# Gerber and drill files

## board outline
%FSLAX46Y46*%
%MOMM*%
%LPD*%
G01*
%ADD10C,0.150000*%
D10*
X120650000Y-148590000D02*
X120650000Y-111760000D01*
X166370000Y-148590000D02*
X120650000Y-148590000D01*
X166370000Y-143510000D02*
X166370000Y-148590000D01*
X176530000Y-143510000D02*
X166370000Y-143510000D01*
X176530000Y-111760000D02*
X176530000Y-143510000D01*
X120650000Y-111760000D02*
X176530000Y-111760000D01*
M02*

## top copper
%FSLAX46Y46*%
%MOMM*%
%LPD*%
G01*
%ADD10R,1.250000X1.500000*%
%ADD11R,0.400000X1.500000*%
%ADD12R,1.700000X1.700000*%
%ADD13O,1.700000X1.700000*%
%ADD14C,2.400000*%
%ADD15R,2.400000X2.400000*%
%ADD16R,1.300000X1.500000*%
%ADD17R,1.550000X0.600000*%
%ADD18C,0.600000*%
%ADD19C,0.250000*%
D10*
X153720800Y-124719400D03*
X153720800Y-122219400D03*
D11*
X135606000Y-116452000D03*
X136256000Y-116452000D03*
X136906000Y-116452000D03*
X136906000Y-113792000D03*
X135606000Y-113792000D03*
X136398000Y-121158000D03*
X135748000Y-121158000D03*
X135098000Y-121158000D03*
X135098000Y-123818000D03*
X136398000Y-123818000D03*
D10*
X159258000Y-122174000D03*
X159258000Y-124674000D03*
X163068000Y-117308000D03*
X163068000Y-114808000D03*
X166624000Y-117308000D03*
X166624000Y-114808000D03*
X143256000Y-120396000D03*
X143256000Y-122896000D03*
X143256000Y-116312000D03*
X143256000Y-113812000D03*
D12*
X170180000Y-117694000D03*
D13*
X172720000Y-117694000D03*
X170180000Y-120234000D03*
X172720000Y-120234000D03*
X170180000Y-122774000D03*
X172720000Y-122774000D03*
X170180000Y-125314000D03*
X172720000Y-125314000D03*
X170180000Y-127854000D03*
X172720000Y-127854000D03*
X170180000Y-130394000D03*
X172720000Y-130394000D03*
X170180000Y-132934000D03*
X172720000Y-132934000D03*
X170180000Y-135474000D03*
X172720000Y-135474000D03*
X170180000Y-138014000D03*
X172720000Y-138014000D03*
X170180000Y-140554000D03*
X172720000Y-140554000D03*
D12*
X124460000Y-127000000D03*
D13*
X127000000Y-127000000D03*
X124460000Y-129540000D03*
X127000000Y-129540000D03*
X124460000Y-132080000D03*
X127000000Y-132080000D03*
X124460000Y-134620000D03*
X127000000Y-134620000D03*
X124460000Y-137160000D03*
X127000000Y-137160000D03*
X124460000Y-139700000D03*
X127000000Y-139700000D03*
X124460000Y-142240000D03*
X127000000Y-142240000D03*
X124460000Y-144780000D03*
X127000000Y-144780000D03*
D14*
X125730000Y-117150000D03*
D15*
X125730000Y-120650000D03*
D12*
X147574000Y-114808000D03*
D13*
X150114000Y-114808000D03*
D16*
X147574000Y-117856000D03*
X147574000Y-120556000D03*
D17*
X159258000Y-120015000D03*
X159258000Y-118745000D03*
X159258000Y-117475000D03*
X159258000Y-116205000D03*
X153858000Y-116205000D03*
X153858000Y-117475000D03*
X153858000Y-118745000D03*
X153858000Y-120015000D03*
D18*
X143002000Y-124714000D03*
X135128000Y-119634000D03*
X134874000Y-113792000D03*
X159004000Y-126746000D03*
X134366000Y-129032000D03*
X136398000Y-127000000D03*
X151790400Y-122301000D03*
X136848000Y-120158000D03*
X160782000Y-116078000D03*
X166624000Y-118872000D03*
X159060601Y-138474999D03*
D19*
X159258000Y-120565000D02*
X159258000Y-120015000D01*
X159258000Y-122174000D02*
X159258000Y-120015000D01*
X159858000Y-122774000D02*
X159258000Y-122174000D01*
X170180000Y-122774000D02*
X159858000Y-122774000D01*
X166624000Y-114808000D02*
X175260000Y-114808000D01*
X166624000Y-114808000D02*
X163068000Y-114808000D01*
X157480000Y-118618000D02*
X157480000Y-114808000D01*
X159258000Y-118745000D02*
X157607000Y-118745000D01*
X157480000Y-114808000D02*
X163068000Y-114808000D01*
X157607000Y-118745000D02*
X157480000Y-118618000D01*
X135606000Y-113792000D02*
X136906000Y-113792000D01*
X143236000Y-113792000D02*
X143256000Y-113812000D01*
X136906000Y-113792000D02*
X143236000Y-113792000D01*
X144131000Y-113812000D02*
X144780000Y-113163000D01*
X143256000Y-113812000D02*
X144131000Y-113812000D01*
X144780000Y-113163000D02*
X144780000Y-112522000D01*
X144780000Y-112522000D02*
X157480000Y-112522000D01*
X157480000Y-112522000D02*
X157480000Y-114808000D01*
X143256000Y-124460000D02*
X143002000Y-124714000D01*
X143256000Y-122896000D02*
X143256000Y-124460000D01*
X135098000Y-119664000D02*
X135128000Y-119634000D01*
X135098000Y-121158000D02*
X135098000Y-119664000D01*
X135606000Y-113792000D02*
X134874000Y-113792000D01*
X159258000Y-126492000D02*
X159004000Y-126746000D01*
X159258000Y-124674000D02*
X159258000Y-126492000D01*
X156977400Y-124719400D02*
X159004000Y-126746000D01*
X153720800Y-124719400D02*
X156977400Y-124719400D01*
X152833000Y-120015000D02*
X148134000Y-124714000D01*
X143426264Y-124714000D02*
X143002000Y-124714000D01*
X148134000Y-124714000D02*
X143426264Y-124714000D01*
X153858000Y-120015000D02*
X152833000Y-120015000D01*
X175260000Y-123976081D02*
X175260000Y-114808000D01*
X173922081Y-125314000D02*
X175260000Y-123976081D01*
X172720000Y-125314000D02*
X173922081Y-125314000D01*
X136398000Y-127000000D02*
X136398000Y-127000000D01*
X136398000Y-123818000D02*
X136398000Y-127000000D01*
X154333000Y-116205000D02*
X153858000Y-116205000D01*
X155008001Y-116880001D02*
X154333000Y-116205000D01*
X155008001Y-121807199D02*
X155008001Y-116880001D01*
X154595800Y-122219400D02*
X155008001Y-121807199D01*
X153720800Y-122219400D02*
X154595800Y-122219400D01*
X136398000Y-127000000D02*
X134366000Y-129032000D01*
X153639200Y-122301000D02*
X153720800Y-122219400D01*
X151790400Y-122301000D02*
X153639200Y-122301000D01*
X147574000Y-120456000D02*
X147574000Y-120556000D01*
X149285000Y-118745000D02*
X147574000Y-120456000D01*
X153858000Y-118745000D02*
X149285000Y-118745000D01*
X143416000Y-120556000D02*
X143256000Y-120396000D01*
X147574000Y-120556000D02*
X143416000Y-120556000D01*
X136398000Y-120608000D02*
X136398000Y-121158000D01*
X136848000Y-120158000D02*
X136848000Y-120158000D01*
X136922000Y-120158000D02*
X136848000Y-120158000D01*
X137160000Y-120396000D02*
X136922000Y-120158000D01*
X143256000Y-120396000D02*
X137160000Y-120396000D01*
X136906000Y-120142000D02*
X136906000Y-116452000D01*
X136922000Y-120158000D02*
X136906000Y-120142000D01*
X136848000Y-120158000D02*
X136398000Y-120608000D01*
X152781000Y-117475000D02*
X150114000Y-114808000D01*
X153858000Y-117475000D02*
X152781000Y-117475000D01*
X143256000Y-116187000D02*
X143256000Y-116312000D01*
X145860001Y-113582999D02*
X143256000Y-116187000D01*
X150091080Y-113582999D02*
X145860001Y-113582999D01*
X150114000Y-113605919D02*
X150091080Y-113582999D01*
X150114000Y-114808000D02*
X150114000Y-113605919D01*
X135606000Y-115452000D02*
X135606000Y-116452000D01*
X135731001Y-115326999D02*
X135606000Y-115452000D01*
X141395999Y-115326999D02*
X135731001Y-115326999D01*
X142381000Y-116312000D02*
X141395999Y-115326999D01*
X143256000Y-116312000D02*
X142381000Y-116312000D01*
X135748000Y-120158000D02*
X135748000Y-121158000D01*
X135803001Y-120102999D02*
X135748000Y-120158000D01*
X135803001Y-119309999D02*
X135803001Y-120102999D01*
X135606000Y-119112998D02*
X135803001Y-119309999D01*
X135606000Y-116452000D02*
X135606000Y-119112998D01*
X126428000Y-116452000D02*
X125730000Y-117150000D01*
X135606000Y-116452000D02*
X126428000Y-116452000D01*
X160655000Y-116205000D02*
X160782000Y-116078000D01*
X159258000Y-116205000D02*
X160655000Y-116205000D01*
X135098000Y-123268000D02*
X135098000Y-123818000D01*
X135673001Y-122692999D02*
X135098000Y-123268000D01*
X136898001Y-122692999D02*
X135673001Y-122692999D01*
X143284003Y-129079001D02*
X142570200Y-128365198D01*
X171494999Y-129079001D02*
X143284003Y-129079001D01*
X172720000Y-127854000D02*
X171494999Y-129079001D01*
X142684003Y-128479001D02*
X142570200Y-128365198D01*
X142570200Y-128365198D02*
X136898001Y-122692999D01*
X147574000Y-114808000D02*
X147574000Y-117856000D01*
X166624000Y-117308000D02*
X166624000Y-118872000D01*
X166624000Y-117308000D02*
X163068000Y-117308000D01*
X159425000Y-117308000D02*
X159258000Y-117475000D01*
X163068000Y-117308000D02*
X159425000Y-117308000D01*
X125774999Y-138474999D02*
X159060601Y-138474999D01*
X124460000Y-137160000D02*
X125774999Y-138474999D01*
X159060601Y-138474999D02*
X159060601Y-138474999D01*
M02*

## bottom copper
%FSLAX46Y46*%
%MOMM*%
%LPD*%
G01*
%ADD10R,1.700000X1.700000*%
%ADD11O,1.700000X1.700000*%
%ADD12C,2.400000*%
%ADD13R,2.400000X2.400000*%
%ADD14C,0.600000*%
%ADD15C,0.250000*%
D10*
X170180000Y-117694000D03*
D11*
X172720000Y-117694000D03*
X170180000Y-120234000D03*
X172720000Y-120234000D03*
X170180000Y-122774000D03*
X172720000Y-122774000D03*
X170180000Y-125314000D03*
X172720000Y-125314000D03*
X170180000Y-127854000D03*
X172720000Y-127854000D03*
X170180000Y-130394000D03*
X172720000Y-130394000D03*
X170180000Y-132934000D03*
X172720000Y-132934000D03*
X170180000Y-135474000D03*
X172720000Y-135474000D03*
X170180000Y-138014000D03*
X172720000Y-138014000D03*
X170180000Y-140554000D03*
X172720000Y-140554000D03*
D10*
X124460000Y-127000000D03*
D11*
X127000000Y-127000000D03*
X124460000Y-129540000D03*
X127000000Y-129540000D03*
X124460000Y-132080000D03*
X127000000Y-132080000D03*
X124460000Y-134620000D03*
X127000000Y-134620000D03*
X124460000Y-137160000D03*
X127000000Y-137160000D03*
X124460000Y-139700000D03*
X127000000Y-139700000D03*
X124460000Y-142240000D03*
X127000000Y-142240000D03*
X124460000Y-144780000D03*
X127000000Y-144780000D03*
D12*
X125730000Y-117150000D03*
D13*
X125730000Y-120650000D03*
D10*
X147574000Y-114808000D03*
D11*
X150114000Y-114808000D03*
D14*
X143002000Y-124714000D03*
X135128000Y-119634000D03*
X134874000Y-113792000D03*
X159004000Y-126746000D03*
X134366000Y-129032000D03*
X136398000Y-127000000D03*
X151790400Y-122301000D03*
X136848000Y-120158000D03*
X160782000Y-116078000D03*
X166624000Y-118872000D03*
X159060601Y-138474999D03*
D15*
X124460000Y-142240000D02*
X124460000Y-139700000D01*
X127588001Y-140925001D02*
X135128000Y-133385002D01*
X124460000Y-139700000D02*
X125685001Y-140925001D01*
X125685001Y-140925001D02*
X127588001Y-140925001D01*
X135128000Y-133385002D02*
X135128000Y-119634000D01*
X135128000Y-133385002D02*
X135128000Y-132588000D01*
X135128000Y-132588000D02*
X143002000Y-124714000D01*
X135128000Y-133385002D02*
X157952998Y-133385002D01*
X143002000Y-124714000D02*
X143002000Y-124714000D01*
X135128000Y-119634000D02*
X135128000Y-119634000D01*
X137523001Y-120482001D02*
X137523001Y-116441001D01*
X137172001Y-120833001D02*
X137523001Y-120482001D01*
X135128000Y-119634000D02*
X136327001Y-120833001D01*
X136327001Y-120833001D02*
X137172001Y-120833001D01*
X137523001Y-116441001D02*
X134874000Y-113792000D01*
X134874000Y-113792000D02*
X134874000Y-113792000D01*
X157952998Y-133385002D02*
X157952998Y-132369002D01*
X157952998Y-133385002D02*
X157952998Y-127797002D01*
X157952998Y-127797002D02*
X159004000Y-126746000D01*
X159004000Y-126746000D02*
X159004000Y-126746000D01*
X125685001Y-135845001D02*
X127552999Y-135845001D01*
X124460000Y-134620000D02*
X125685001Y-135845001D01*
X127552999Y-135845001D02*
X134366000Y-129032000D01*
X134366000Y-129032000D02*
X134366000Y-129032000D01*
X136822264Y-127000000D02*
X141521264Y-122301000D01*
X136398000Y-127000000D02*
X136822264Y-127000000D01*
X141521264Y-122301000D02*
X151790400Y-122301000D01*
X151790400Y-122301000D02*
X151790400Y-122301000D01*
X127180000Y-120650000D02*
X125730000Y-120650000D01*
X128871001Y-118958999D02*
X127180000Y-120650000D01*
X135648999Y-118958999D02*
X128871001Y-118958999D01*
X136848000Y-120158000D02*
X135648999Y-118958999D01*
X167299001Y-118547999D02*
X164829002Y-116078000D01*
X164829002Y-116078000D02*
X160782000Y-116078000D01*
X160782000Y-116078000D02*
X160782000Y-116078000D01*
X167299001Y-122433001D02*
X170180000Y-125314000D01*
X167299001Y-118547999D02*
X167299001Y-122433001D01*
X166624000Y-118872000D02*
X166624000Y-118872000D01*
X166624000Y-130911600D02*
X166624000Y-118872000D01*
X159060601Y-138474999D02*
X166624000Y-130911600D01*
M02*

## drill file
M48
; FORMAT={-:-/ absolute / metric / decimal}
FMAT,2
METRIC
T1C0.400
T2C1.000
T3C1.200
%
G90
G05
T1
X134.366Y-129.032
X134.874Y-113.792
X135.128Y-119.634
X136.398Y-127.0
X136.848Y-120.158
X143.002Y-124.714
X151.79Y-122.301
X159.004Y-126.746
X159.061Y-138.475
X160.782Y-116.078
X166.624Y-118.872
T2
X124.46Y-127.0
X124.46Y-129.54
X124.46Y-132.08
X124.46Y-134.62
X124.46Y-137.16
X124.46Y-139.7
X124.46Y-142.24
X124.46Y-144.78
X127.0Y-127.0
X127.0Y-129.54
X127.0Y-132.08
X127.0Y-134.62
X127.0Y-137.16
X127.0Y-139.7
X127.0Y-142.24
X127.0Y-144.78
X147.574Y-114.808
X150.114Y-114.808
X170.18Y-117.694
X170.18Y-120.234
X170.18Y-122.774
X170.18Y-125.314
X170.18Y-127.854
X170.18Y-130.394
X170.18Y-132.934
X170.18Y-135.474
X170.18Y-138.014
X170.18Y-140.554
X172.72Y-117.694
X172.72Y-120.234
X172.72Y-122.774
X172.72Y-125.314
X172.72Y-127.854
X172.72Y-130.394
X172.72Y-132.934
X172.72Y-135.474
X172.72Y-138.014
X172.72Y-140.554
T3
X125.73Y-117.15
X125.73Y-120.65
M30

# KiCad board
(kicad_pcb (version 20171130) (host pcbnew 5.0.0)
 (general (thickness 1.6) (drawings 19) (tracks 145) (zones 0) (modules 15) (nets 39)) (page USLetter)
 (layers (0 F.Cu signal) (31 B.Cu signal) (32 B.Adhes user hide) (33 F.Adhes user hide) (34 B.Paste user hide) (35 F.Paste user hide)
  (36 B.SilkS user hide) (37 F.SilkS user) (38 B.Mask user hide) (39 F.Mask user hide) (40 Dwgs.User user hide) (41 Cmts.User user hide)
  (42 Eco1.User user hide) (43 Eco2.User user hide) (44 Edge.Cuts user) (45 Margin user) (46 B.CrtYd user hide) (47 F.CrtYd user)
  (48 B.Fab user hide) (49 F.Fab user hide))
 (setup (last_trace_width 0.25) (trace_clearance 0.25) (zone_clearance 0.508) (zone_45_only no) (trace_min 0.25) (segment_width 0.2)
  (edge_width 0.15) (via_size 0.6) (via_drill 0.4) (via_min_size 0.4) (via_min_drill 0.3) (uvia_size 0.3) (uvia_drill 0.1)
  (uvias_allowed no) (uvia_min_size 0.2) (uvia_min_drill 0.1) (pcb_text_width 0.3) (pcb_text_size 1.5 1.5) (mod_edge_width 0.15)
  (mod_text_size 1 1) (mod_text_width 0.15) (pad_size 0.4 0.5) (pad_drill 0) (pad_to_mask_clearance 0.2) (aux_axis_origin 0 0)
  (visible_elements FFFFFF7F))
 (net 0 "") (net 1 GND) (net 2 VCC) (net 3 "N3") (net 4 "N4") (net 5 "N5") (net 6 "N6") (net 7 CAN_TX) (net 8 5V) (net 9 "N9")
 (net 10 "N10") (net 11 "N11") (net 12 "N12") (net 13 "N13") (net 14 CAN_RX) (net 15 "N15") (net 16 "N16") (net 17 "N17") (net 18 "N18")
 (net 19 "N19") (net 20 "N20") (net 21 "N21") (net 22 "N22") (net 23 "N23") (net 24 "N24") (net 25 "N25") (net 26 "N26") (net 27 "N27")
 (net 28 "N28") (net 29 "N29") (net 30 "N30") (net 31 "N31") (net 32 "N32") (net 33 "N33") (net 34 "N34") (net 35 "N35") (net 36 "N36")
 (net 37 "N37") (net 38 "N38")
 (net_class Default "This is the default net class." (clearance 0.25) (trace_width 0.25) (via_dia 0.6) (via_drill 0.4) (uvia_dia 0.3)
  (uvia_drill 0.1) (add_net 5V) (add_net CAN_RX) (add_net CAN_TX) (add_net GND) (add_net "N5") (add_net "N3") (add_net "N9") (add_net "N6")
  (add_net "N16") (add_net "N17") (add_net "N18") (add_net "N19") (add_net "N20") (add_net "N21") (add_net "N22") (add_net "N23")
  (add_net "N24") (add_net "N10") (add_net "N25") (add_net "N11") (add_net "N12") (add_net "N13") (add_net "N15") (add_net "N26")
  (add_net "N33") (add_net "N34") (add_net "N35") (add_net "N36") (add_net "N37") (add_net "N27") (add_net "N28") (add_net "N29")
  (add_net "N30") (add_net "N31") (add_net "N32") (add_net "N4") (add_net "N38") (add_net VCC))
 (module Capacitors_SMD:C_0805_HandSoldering (layer F.Cu) (at 153.7208 123.4694 90)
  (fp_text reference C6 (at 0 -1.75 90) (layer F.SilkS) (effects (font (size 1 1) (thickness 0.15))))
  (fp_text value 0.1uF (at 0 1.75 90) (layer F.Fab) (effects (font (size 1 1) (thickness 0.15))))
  (pad 1 smd rect (at -1.25 0 90) (size 1.5 1.25) (layers F.Cu F.Paste F.Mask) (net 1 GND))
  (pad 2 smd rect (at 1.25 0 90) (size 1.5 1.25) (layers F.Cu F.Paste F.Mask) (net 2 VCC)))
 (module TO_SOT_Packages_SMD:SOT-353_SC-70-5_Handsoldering (layer F.Cu) (at 136.256 115.122 90)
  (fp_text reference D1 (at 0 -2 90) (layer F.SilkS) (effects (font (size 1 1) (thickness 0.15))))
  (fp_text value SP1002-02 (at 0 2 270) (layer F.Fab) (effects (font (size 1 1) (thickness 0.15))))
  (pad 1 smd rect (at -1.33 -0.65 90) (size 1.5 0.4) (layers F.Cu F.Paste F.Mask) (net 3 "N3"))
  (pad 2 smd rect (at -1.33 0 90) (size 1.5 0.4) (layers F.Cu F.Paste F.Mask) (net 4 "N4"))
  (pad 3 smd rect (at -1.33 0.65 90) (size 1.5 0.4) (layers F.Cu F.Paste F.Mask) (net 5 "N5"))
  (pad 4 smd rect (at 1.33 0.65 90) (size 1.5 0.4) (layers F.Cu F.Paste F.Mask) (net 1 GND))
  (pad 5 smd rect (at 1.33 -0.65 90) (size 1.5 0.4) (layers F.Cu F.Paste F.Mask) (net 1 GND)))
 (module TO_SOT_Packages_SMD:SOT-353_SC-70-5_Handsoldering (layer F.Cu) (at 135.748 122.488 270)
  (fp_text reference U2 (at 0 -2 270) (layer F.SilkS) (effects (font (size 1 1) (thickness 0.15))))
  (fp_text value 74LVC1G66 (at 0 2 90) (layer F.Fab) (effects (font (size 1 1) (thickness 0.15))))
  (pad 1 smd rect (at -1.33 -0.65 270) (size 1.5 0.4) (layers F.Cu F.Paste F.Mask) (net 5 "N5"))
  (pad 2 smd rect (at -1.33 0 270) (size 1.5 0.4) (layers F.Cu F.Paste F.Mask) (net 3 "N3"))
  (pad 3 smd rect (at -1.33 0.65 270) (size 1.5 0.4) (layers F.Cu F.Paste F.Mask) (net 1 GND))
  (pad 4 smd rect (at 1.33 0.65 270) (size 1.5 0.4) (layers F.Cu F.Paste F.Mask) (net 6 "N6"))
  (pad 5 smd rect (at 1.33 -0.65 270) (size 1.5 0.4) (layers F.Cu F.Paste F.Mask) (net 2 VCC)))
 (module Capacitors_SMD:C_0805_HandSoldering (layer F.Cu) (at 159.258 123.424 270)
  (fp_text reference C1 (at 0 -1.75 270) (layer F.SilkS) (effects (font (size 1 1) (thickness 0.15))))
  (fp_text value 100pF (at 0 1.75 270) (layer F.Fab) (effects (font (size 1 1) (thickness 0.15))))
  (pad 1 smd rect (at -1.25 0 270) (size 1.5 1.25) (layers F.Cu F.Paste F.Mask) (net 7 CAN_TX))
  (pad 2 smd rect (at 1.25 0 270) (size 1.5 1.25) (layers F.Cu F.Paste F.Mask) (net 1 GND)))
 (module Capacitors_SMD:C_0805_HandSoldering (layer F.Cu) (at 163.068 116.058 90)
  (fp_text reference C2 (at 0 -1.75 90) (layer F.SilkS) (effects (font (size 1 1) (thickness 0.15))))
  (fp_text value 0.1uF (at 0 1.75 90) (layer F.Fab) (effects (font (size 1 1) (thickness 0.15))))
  (pad 1 smd rect (at -1.25 0 90) (size 1.5 1.25) (layers F.Cu F.Paste F.Mask) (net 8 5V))
  (pad 2 smd rect (at 1.25 0 90) (size 1.5 1.25) (layers F.Cu F.Paste F.Mask) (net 1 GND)))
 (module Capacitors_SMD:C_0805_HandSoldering (layer F.Cu) (at 166.624 116.058 90)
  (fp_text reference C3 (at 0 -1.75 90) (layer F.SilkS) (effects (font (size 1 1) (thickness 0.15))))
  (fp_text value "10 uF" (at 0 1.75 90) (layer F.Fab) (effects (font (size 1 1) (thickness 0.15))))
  (pad 1 smd rect (at -1.25 0 90) (size 1.5 1.25) (layers F.Cu F.Paste F.Mask) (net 8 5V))
  (pad 2 smd rect (at 1.25 0 90) (size 1.5 1.25) (layers F.Cu F.Paste F.Mask) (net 1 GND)))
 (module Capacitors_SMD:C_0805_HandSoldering (layer F.Cu) (at 143.256 121.646 270)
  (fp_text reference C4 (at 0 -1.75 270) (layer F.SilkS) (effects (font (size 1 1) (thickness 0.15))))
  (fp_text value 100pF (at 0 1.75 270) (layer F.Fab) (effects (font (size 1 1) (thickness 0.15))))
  (pad 1 smd rect (at -1.25 0 270) (size 1.5 1.25) (layers F.Cu F.Paste F.Mask) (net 5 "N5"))
  (pad 2 smd rect (at 1.25 0 270) (size 1.5 1.25) (layers F.Cu F.Paste F.Mask) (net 1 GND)))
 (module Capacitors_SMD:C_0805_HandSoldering (layer F.Cu) (at 143.256 115.062 90)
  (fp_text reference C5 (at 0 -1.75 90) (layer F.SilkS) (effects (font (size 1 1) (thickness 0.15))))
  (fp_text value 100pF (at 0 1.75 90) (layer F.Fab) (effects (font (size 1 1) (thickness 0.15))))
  (pad 1 smd rect (at -1.25 0 90) (size 1.5 1.25) (layers F.Cu F.Paste F.Mask) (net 3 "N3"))
  (pad 2 smd rect (at 1.25 0 90) (size 1.5 1.25) (layers F.Cu F.Paste F.Mask) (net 1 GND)))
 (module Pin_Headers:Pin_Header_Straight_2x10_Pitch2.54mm (layer F.Cu) (at 170.18 117.694)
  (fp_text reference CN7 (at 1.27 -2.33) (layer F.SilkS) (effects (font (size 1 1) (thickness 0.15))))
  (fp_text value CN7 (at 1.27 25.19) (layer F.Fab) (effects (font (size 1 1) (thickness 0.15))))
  (pad 1 thru_hole rect (at 0 0) (size 1.7 1.7) (drill 1) (layers *.Cu *.Mask) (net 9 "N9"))
  (pad 2 thru_hole oval (at 2.54 0) (size 1.7 1.7) (drill 1) (layers *.Cu *.Mask) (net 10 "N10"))
  (pad 3 thru_hole oval (at 0 2.54) (size 1.7 1.7) (drill 1) (layers *.Cu *.Mask) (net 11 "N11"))
  (pad 4 thru_hole oval (at 2.54 2.54) (size 1.7 1.7) (drill 1) (layers *.Cu *.Mask) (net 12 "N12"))
  (pad 5 thru_hole oval (at 0 5.08) (size 1.7 1.7) (drill 1) (layers *.Cu *.Mask) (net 7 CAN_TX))
  (pad 6 thru_hole oval (at 2.54 5.08) (size 1.7 1.7) (drill 1) (layers *.Cu *.Mask) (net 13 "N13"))
  (pad 7 thru_hole oval (at 0 7.62) (size 1.7 1.7) (drill 1) (layers *.Cu *.Mask) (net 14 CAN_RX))
  (pad 8 thru_hole oval (at 2.54 7.62) (size 1.7 1.7) (drill 1) (layers *.Cu *.Mask) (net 1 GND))
  (pad 9 thru_hole oval (at 0 10.16) (size 1.7 1.7) (drill 1) (layers *.Cu *.Mask) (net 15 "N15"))
  (pad 10 thru_hole oval (at 2.54 10.16) (size 1.7 1.7) (drill 1) (layers *.Cu *.Mask) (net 6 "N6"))
  (pad 11 thru_hole oval (at 0 12.7) (size 1.7 1.7) (drill 1) (layers *.Cu *.Mask) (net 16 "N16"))
  (pad 12 thru_hole oval (at 2.54 12.7) (size 1.7 1.7) (drill 1) (layers *.Cu *.Mask) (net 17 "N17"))
  (pad 13 thru_hole oval (at 0 15.24) (size 1.7 1.7) (drill 1) (layers *.Cu *.Mask) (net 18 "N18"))
  (pad 14 thru_hole oval (at 2.54 15.24) (size 1.7 1.7) (drill 1) (layers *.Cu *.Mask) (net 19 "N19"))
  (pad 15 thru_hole oval (at 0 17.78) (size 1.7 1.7) (drill 1) (layers *.Cu *.Mask) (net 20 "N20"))
  (pad 16 thru_hole oval (at 2.54 17.78) (size 1.7 1.7) (drill 1) (layers *.Cu *.Mask) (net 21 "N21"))
  (pad 17 thru_hole oval (at 0 20.32) (size 1.7 1.7) (drill 1) (layers *.Cu *.Mask) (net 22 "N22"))
  (pad 18 thru_hole oval (at 2.54 20.32) (size 1.7 1.7) (drill 1) (layers *.Cu *.Mask) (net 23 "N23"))
  (pad 19 thru_hole oval (at 0 22.86) (size 1.7 1.7) (drill 1) (layers *.Cu *.Mask) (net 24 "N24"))
  (pad 20 thru_hole oval (at 2.54 22.86) (size 1.7 1.7) (drill 1) (layers *.Cu *.Mask) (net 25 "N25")))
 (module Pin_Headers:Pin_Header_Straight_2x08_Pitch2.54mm (layer F.Cu) (at 124.46 127)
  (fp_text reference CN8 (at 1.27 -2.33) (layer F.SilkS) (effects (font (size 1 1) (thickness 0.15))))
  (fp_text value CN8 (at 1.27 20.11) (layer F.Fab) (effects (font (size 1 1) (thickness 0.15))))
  (pad 1 thru_hole rect (at 0 0) (size 1.7 1.7) (drill 1) (layers *.Cu *.Mask) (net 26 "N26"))
  (pad 2 thru_hole oval (at 2.54 0) (size 1.7 1.7) (drill 1) (layers *.Cu *.Mask) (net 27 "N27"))
  (pad 3 thru_hole oval (at 0 2.54) (size 1.7 1.7) (drill 1) (layers *.Cu *.Mask) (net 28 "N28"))
  (pad 4 thru_hole oval (at 2.54 2.54) (size 1.7 1.7) (drill 1) (layers *.Cu *.Mask) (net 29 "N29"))
  (pad 5 thru_hole oval (at 0 5.08) (size 1.7 1.7) (drill 1) (layers *.Cu *.Mask) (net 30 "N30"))
  (pad 6 thru_hole oval (at 2.54 5.08) (size 1.7 1.7) (drill 1) (layers *.Cu *.Mask) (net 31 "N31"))
  (pad 7 thru_hole oval (at 0 7.62) (size 1.7 1.7) (drill 1) (layers *.Cu *.Mask) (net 2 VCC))
  (pad 8 thru_hole oval (at 2.54 7.62) (size 1.7 1.7) (drill 1) (layers *.Cu *.Mask) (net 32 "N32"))
  (pad 9 thru_hole oval (at 0 10.16) (size 1.7 1.7) (drill 1) (layers *.Cu *.Mask) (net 8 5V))
  (pad 10 thru_hole oval (at 2.54 10.16) (size 1.7 1.7) (drill 1) (layers *.Cu *.Mask) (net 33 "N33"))
  (pad 11 thru_hole oval (at 0 12.7) (size 1.7 1.7) (drill 1) (layers *.Cu *.Mask) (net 1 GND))
  (pad 12 thru_hole oval (at 2.54 12.7) (size 1.7 1.7) (drill 1) (layers *.Cu *.Mask) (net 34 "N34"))
  (pad 13 thru_hole oval (at 0 15.24) (size 1.7 1.7) (drill 1) (layers *.Cu *.Mask) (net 1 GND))
  (pad 14 thru_hole oval (at 2.54 15.24) (size 1.7 1.7) (drill 1) (layers *.Cu *.Mask) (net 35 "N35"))
  (pad 15 thru_hole oval (at 0 17.78) (size 1.7 1.7) (drill 1) (layers *.Cu *.Mask) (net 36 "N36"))
  (pad 16 thru_hole oval (at 2.54 17.78) (size 1.7 1.7) (drill 1) (layers *.Cu *.Mask) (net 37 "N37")))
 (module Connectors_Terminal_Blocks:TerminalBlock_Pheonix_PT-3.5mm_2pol (layer F.Cu) (at 125.73 120.65 90)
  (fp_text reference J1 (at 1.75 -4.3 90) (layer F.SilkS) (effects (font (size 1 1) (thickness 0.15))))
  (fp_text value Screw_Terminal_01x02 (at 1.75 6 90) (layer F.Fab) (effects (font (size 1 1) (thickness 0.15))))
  (pad 2 thru_hole circle (at 3.5 0 90) (size 2.4 2.4) (drill 1.2) (layers *.Cu *.Mask) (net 3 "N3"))
  (pad 1 thru_hole rect (at 0 0 90) (size 2.4 2.4) (drill 1.2) (layers *.Cu *.Mask) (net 5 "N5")))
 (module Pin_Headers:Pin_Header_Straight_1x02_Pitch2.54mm (layer F.Cu) (at 147.574 114.808 90)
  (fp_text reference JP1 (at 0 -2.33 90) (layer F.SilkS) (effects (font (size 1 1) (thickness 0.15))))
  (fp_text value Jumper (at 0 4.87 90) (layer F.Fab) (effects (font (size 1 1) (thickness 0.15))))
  (pad 1 thru_hole rect (at 0 0 90) (size 1.7 1.7) (drill 1) (layers *.Cu *.Mask) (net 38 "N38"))
  (pad 2 thru_hole oval (at 0 2.54 90) (size 1.7 1.7) (drill 1) (layers *.Cu *.Mask) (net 3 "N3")))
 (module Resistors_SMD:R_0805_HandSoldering (layer F.Cu) (at 147.574 119.206 270)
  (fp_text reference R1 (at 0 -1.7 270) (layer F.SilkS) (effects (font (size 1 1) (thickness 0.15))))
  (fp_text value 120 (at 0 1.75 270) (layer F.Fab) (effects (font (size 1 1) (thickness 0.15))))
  (pad 1 smd rect (at -1.35 0 270) (size 1.5 1.3) (layers F.Cu F.Paste F.Mask) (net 38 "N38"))
  (pad 2 smd rect (at 1.35 0 270) (size 1.5 1.3) (layers F.Cu F.Paste F.Mask) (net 5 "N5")))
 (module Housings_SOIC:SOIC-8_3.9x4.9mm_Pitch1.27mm (layer F.Cu) (at 156.558 118.11 180)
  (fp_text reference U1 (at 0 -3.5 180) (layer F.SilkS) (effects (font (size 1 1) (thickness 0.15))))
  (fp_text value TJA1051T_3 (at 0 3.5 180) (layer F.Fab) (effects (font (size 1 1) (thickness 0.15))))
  (pad 1 smd rect (at -2.7 -1.905 180) (size 1.55 0.6) (layers F.Cu F.Paste F.Mask) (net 7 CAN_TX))
  (pad 2 smd rect (at -2.7 -0.635 180) (size 1.55 0.6) (layers F.Cu F.Paste F.Mask) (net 1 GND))
  (pad 3 smd rect (at -2.7 0.635 180) (size 1.55 0.6) (layers F.Cu F.Paste F.Mask) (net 8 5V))
  (pad 4 smd rect (at -2.7 1.905 180) (size 1.55 0.6) (layers F.Cu F.Paste F.Mask) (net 14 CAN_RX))
  (pad 5 smd rect (at 2.7 1.905 180) (size 1.55 0.6) (layers F.Cu F.Paste F.Mask) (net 2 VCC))
  (pad 6 smd rect (at 2.7 0.635 180) (size 1.55 0.6) (layers F.Cu F.Paste F.Mask) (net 3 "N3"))
  (pad 7 smd rect (at 2.7 -0.635 180) (size 1.55 0.6) (layers F.Cu F.Paste F.Mask) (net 5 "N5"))
  (pad 8 smd rect (at 2.7 -1.905 180) (size 1.55 0.6) (layers F.Cu F.Paste F.Mask) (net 1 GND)))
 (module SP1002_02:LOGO (layer B.Cu) (at 147.32 134.2898)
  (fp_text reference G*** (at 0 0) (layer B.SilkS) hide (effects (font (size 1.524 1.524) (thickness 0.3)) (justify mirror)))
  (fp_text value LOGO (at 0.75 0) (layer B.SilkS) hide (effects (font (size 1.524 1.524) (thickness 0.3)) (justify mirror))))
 (gr_line (start 120.65 148.59) (end 120.65 111.76) (angle 90) (layer Edge.Cuts) (width 0.15))
 (gr_line (start 166.37 148.59) (end 120.65 148.59) (angle 90) (layer Edge.Cuts) (width 0.15))
 (gr_line (start 166.37 143.51) (end 166.37 148.59) (angle 90) (layer Edge.Cuts) (width 0.15))
 (gr_line (start 176.53 143.51) (end 166.37 143.51) (angle 90) (layer Edge.Cuts) (width 0.15))
 (gr_line (start 176.53 111.76) (end 176.53 143.51) (angle 90) (layer Edge.Cuts) (width 0.15))
 (gr_line (start 120.65 111.76) (end 176.53 111.76) (angle 90) (layer Edge.Cuts) (width 0.15))
 (segment (start 159.258 120.565) (end 159.258 120.015) (width 0.25) (layer F.Cu) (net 7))
 (segment (start 159.258 122.174) (end 159.258 120.015) (width 0.25) (layer F.Cu) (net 7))
 (segment (start 159.858 122.774) (end 159.258 122.174) (width 0.25) (layer F.Cu) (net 7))
 (segment (start 170.18 122.774) (end 159.858 122.774) (width 0.25) (layer F.Cu) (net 7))
 (segment (start 124.46 142.24) (end 124.46 139.7) (width 0.25) (layer B.Cu) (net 1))
 (segment (start 166.624 114.808) (end 175.26 114.808) (width 0.25) (layer F.Cu) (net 1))
 (segment (start 166.624 114.808) (end 163.068 114.808) (width 0.25) (layer F.Cu) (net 1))
 (segment (start 157.48 118.618) (end 157.48 114.808) (width 0.25) (layer F.Cu) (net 1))
 (segment (start 159.258 118.745) (end 157.607 118.745) (width 0.25) (layer F.Cu) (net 1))
 (segment (start 157.48 114.808) (end 163.068 114.808) (width 0.25) (layer F.Cu) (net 1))
 (segment (start 157.607 118.745) (end 157.48 118.618) (width 0.25) (layer F.Cu) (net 1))
 (segment (start 135.606 113.792) (end 136.906 113.792) (width 0.25) (layer F.Cu) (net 1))
 (segment (start 143.236 113.792) (end 143.256 113.812) (width 0.25) (layer F.Cu) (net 1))
 (segment (start 136.906 113.792) (end 143.236 113.792) (width 0.25) (layer F.Cu) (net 1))
 (segment (start 144.131 113.812) (end 144.78 113.163) (width 0.25) (layer F.Cu) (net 1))
 (segment (start 143.256 113.812) (end 144.131 113.812) (width 0.25) (layer F.Cu) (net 1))
 (segment (start 144.78 113.163) (end 144.78 112.522) (width 0.25) (layer F.Cu) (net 1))
 (segment (start 144.78 112.522) (end 157.48 112.522) (width 0.25) (layer F.Cu) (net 1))
 (segment (start 157.48 112.522) (end 157.48 114.808) (width 0.25) (layer F.Cu) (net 1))
 (segment (start 127.588001 140.925001) (end 135.128 133.385002) (width 0.25) (layer B.Cu) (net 1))
 (segment (start 124.46 139.7) (end 125.685001 140.925001) (width 0.25) (layer B.Cu) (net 1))
 (segment (start 125.685001 140.925001) (end 127.588001 140.925001) (width 0.25) (layer B.Cu) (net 1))
 (segment (start 135.128 133.385002) (end 135.128 119.634) (width 0.25) (layer B.Cu) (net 1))
 (segment (start 135.128 133.385002) (end 135.128 132.588) (width 0.25) (layer B.Cu) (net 1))
 (segment (start 135.128 132.588) (end 143.002 124.714) (width 0.25) (layer B.Cu) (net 1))
 (segment (start 135.128 133.385002) (end 157.952998 133.385002) (width 0.25) (layer B.Cu) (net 1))
 (segment (start 143.002 124.714) (end 143.002 124.714) (width 0.25) (layer B.Cu) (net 1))
 (via (at 143.002 124.714) (size 0.6) (drill 0.4) (layers F.Cu B.Cu) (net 1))
 (segment (start 135.128 119.634) (end 135.128 119.634) (width 0.25) (layer B.Cu) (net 1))
 (via (at 135.128 119.634) (size 0.6) (drill 0.4) (layers F.Cu B.Cu) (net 1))
 (segment (start 143.256 124.46) (end 143.002 124.714) (width 0.25) (layer F.Cu) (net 1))
 (segment (start 143.256 122.896) (end 143.256 124.46) (width 0.25) (layer F.Cu) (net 1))
 (segment (start 135.098 119.664) (end 135.128 119.634) (width 0.25) (layer F.Cu) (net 1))
 (segment (start 135.098 121.158) (end 135.098 119.664) (width 0.25) (layer F.Cu) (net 1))
 (segment (start 137.523001 120.482001) (end 137.523001 116.441001) (width 0.25) (layer B.Cu) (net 1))
 (segment (start 137.172001 120.833001) (end 137.523001 120.482001) (width 0.25) (layer B.Cu) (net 1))
 (segment (start 135.128 119.634) (end 136.327001 120.833001) (width 0.25) (layer B.Cu) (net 1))
 (segment (start 136.327001 120.833001) (end 137.172001 120.833001) (width 0.25) (layer B.Cu) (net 1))
 (segment (start 137.523001 116.441001) (end 134.874 113.792) (width 0.25) (layer B.Cu) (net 1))
 (segment (start 134.874 113.792) (end 134.874 113.792) (width 0.25) (layer B.Cu) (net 1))
 (via (at 134.874 113.792) (size 0.6) (drill 0.4) (layers F.Cu B.Cu) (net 1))
 (segment (start 135.606 113.792) (end 134.874 113.792) (width 0.25) (layer F.Cu) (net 1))
 (segment (start 157.952998 133.385002) (end 157.952998 132.369002) (width 0.25) (layer B.Cu) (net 1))
 (segment (start 157.952998 133.385002) (end 157.952998 127.797002) (width 0.25) (layer B.Cu) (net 1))
 (segment (start 157.952998 127.797002) (end 159.004 126.746) (width 0.25) (layer B.Cu) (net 1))
 (segment (start 159.004 126.746) (end 159.004 126.746) (width 0.25) (layer B.Cu) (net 1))
 (via (at 159.004 126.746) (size 0.6) (drill 0.4) (layers F.Cu B.Cu) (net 1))
 (segment (start 159.258 126.492) (end 159.004 126.746) (width 0.25) (layer F.Cu) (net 1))
 (segment (start 159.258 124.674) (end 159.258 126.492) (width 0.25) (layer F.Cu) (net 1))
 (segment (start 156.9774 124.7194) (end 159.004 126.746) (width 0.25) (layer F.Cu) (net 1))
 (segment (start 153.7208 124.7194) (end 156.9774 124.7194) (width 0.25) (layer F.Cu) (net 1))
 (segment (start 152.833 120.015) (end 148.134 124.714) (width 0.25) (layer F.Cu) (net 1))
 (segment (start 143.426264 124.714) (end 143.002 124.714) (width 0.25) (layer F.Cu) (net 1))
 (segment (start 148.134 124.714) (end 143.426264 124.714) (width 0.25) (layer F.Cu) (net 1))
 (segment (start 153.858 120.015) (end 152.833 120.015) (width 0.25) (layer F.Cu) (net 1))
 (segment (start 175.26 123.976081) (end 175.26 114.808) (width 0.25) (layer F.Cu) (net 1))
 (segment (start 173.922081 125.314) (end 175.26 123.976081) (width 0.25) (layer F.Cu) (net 1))
 (segment (start 172.72 125.314) (end 173.922081 125.314) (width 0.25) (layer F.Cu) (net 1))
 (segment (start 125.685001 135.845001) (end 127.552999 135.845001) (width 0.25) (layer B.Cu) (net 2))
 (segment (start 124.46 134.62) (end 125.685001 135.845001) (width 0.25) (layer B.Cu) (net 2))
 (segment (start 127.552999 135.845001) (end 134.366 129.032) (width 0.25) (layer B.Cu) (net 2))
 (segment (start 134.366 129.032) (end 134.366 129.032) (width 0.25) (layer B.Cu) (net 2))
 (via (at 134.366 129.032) (size 0.6) (drill 0.4) (layers F.Cu B.Cu) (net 2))
 (segment (start 136.398 127) (end 136.398 127) (width 0.25) (layer F.Cu) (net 2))
 (segment (start 136.398 123.818) (end 136.398 127) (width 0.25) (layer F.Cu) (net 2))
 (segment (start 154.333 116.205) (end 153.858 116.205) (width 0.25) (layer F.Cu) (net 2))
 (segment (start 155.008001 116.880001) (end 154.333 116.205) (width 0.25) (layer F.Cu) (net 2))
 (segment (start 155.008001 121.807199) (end 155.008001 116.880001) (width 0.25) (layer F.Cu) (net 2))
 (segment (start 154.5958 122.2194) (end 155.008001 121.807199) (width 0.25) (layer F.Cu) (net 2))
 (segment (start 153.7208 122.2194) (end 154.5958 122.2194) (width 0.25) (layer F.Cu) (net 2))
 (segment (start 136.398 127) (end 134.366 129.032) (width 0.25) (layer F.Cu) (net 2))
 (via (at 136.398 127) (size 0.6) (drill 0.4) (layers F.Cu B.Cu) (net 2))
 (segment (start 136.822264 127) (end 141.521264 122.301) (width 0.25) (layer B.Cu) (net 2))
 (segment (start 136.398 127) (end 136.822264 127) (width 0.25) (layer B.Cu) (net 2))
 (segment (start 141.521264 122.301) (end 151.7904 122.301) (width 0.25) (layer B.Cu) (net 2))
 (segment (start 151.7904 122.301) (end 151.7904 122.301) (width 0.25) (layer B.Cu) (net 2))
 (via (at 151.7904 122.301) (size 0.6) (drill 0.4) (layers F.Cu B.Cu) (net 2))
 (segment (start 153.6392 122.301) (end 153.7208 122.2194) (width 0.25) (layer F.Cu) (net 2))
 (segment (start 151.7904 122.301) (end 153.6392 122.301) (width 0.25) (layer F.Cu) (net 2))
 (segment (start 147.574 120.456) (end 147.574 120.556) (width 0.25) (layer F.Cu) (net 5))
 (segment (start 149.285 118.745) (end 147.574 120.456) (width 0.25) (layer F.Cu) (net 5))
 (segment (start 153.858 118.745) (end 149.285 118.745) (width 0.25) (layer F.Cu) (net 5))
 (segment (start 143.416 120.556) (end 143.256 120.396) (width 0.25) (layer F.Cu) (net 5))
 (segment (start 147.574 120.556) (end 143.416 120.556) (width 0.25) (layer F.Cu) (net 5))
 (segment (start 136.398 120.608) (end 136.398 121.158) (width 0.25) (layer F.Cu) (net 5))
 (segment (start 136.848 120.158) (end 136.848 120.158) (width 0.25) (layer F.Cu) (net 5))
 (segment (start 136.922 120.158) (end 136.848 120.158) (width 0.25) (layer F.Cu) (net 5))
 (segment (start 137.16 120.396) (end 136.922 120.158) (width 0.25) (layer F.Cu) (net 5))
 (segment (start 143.256 120.396) (end 137.16 120.396) (width 0.25) (layer F.Cu) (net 5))
 (segment (start 136.906 120.142) (end 136.906 116.452) (width 0.25) (layer F.Cu) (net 5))
 (segment (start 136.922 120.158) (end 136.906 120.142) (width 0.25) (layer F.Cu) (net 5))
 (segment (start 136.848 120.158) (end 136.398 120.608) (width 0.25) (layer F.Cu) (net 5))
 (via (at 136.848 120.158) (size 0.6) (drill 0.4) (layers F.Cu B.Cu) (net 5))
 (segment (start 127.18 120.65) (end 125.73 120.65) (width 0.25) (layer B.Cu) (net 5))
 (segment (start 128.871001 118.958999) (end 127.18 120.65) (width 0.25) (layer B.Cu) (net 5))
 (segment (start 135.648999 118.958999) (end 128.871001 118.958999) (width 0.25) (layer B.Cu) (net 5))
 (segment (start 136.848 120.158) (end 135.648999 118.958999) (width 0.25) (layer B.Cu) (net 5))
 (segment (start 152.781 117.475) (end 150.114 114.808) (width 0.25) (layer F.Cu) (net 3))
 (segment (start 153.858 117.475) (end 152.781 117.475) (width 0.25) (layer F.Cu) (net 3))
 (segment (start 143.256 116.187) (end 143.256 116.312) (width 0.25) (layer F.Cu) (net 3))
 (segment (start 145.860001 113.582999) (end 143.256 116.187) (width 0.25) (layer F.Cu) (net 3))
 (segment (start 150.09108 113.582999) (end 145.860001 113.582999) (width 0.25) (layer F.Cu) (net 3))
 (segment (start 150.114 113.605919) (end 150.09108 113.582999) (width 0.25) (layer F.Cu) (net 3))
 (segment (start 150.114 114.808) (end 150.114 113.605919) (width 0.25) (layer F.Cu) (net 3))
 (segment (start 135.606 115.452) (end 135.606 116.452) (width 0.25) (layer F.Cu) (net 3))
 (segment (start 135.731001 115.326999) (end 135.606 115.452) (width 0.25) (layer F.Cu) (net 3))
 (segment (start 141.395999 115.326999) (end 135.731001 115.326999) (width 0.25) (layer F.Cu) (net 3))
 (segment (start 142.381 116.312) (end 141.395999 115.326999) (width 0.25) (layer F.Cu) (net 3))
 (segment (start 143.256 116.312) (end 142.381 116.312) (width 0.25) (layer F.Cu) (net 3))
 (segment (start 135.748 120.158) (end 135.748 121.158) (width 0.25) (layer F.Cu) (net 3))
 (segment (start 135.803001 120.102999) (end 135.748 120.158) (width 0.25) (layer F.Cu) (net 3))
 (segment (start 135.803001 119.309999) (end 135.803001 120.102999) (width 0.25) (layer F.Cu) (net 3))
 (segment (start 135.606 119.112998) (end 135.803001 119.309999) (width 0.25) (layer F.Cu) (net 3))
 (segment (start 135.606 116.452) (end 135.606 119.112998) (width 0.25) (layer F.Cu) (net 3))
 (segment (start 126.428 116.452) (end 125.73 117.15) (width 0.25) (layer F.Cu) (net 3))
 (segment (start 135.606 116.452) (end 126.428 116.452) (width 0.25) (layer F.Cu) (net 3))
 (segment (start 167.299001 118.547999) (end 164.829002 116.078) (width 0.25) (layer B.Cu) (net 14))
 (segment (start 164.829002 116.078) (end 160.782 116.078) (width 0.25) (layer B.Cu) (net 14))
 (segment (start 160.782 116.078) (end 160.782 116.078) (width 0.25) (layer B.Cu) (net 14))
 (via (at 160.782 116.078) (size 0.6) (drill 0.4) (layers F.Cu B.Cu) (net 14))
 (segment (start 160.655 116.205) (end 160.782 116.078) (width 0.25) (layer F.Cu) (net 14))
 (segment (start 159.258 116.205) (end 160.655 116.205) (width 0.25) (layer F.Cu) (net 14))
 (segment (start 167.299001 122.433001) (end 170.18 125.314) (width 0.25) (layer B.Cu) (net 14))
 (segment (start 167.299001 118.547999) (end 167.299001 122.433001) (width 0.25) (layer B.Cu) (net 14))
 (segment (start 135.098 123.268) (end 135.098 123.818) (width 0.25) (layer F.Cu) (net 6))
 (segment (start 135.673001 122.692999) (end 135.098 123.268) (width 0.25) (layer F.Cu) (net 6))
 (segment (start 136.898001 122.692999) (end 135.673001 122.692999) (width 0.25) (layer F.Cu) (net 6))
 (segment (start 143.284003 129.079001) (end 142.5702 128.365198) (width 0.25) (layer F.Cu) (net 6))
 (segment (start 171.494999 129.079001) (end 143.284003 129.079001) (width 0.25) (layer F.Cu) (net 6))
 (segment (start 172.72 127.854) (end 171.494999 129.079001) (width 0.25) (layer F.Cu) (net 6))
 (segment (start 142.684003 128.479001) (end 142.5702 128.365198) (width 0.25) (layer F.Cu) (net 6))
 (segment (start 142.5702 128.365198) (end 136.898001 122.692999) (width 0.25) (layer F.Cu) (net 6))
 (segment (start 147.574 114.808) (end 147.574 117.856) (width 0.25) (layer F.Cu) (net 38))
 (segment (start 166.624 118.872) (end 166.624 118.872) (width 0.25) (layer B.Cu) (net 8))
 (via (at 166.624 118.872) (size 0.6) (drill 0.4) (layers F.Cu B.Cu) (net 8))
 (segment (start 166.624 117.308) (end 166.624 118.872) (width 0.25) (layer F.Cu) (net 8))
 (segment (start 166.624 117.308) (end 163.068 117.308) (width 0.25) (layer F.Cu) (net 8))
 (segment (start 159.425 117.308) (end 159.258 117.475) (width 0.25) (layer F.Cu) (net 8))
 (segment (start 163.068 117.308) (end 159.425 117.308) (width 0.25) (layer F.Cu) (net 8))
 (segment (start 125.774999 138.474999) (end 159.060601 138.474999) (width 0.25) (layer F.Cu) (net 8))
 (segment (start 124.46 137.16) (end 125.774999 138.474999) (width 0.25) (layer F.Cu) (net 8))
 (segment (start 159.060601 138.474999) (end 159.060601 138.474999) (width 0.25) (layer F.Cu) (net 8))
 (via (at 159.060601 138.474999) (size 0.6) (drill 0.4) (layers F.Cu B.Cu) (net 8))
 (segment (start 166.624 130.9116) (end 166.624 118.872) (width 0.25) (layer B.Cu) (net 8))
 (segment (start 159.060601 138.474999) (end 166.624 130.9116) (width 0.25) (layer B.Cu) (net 8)))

